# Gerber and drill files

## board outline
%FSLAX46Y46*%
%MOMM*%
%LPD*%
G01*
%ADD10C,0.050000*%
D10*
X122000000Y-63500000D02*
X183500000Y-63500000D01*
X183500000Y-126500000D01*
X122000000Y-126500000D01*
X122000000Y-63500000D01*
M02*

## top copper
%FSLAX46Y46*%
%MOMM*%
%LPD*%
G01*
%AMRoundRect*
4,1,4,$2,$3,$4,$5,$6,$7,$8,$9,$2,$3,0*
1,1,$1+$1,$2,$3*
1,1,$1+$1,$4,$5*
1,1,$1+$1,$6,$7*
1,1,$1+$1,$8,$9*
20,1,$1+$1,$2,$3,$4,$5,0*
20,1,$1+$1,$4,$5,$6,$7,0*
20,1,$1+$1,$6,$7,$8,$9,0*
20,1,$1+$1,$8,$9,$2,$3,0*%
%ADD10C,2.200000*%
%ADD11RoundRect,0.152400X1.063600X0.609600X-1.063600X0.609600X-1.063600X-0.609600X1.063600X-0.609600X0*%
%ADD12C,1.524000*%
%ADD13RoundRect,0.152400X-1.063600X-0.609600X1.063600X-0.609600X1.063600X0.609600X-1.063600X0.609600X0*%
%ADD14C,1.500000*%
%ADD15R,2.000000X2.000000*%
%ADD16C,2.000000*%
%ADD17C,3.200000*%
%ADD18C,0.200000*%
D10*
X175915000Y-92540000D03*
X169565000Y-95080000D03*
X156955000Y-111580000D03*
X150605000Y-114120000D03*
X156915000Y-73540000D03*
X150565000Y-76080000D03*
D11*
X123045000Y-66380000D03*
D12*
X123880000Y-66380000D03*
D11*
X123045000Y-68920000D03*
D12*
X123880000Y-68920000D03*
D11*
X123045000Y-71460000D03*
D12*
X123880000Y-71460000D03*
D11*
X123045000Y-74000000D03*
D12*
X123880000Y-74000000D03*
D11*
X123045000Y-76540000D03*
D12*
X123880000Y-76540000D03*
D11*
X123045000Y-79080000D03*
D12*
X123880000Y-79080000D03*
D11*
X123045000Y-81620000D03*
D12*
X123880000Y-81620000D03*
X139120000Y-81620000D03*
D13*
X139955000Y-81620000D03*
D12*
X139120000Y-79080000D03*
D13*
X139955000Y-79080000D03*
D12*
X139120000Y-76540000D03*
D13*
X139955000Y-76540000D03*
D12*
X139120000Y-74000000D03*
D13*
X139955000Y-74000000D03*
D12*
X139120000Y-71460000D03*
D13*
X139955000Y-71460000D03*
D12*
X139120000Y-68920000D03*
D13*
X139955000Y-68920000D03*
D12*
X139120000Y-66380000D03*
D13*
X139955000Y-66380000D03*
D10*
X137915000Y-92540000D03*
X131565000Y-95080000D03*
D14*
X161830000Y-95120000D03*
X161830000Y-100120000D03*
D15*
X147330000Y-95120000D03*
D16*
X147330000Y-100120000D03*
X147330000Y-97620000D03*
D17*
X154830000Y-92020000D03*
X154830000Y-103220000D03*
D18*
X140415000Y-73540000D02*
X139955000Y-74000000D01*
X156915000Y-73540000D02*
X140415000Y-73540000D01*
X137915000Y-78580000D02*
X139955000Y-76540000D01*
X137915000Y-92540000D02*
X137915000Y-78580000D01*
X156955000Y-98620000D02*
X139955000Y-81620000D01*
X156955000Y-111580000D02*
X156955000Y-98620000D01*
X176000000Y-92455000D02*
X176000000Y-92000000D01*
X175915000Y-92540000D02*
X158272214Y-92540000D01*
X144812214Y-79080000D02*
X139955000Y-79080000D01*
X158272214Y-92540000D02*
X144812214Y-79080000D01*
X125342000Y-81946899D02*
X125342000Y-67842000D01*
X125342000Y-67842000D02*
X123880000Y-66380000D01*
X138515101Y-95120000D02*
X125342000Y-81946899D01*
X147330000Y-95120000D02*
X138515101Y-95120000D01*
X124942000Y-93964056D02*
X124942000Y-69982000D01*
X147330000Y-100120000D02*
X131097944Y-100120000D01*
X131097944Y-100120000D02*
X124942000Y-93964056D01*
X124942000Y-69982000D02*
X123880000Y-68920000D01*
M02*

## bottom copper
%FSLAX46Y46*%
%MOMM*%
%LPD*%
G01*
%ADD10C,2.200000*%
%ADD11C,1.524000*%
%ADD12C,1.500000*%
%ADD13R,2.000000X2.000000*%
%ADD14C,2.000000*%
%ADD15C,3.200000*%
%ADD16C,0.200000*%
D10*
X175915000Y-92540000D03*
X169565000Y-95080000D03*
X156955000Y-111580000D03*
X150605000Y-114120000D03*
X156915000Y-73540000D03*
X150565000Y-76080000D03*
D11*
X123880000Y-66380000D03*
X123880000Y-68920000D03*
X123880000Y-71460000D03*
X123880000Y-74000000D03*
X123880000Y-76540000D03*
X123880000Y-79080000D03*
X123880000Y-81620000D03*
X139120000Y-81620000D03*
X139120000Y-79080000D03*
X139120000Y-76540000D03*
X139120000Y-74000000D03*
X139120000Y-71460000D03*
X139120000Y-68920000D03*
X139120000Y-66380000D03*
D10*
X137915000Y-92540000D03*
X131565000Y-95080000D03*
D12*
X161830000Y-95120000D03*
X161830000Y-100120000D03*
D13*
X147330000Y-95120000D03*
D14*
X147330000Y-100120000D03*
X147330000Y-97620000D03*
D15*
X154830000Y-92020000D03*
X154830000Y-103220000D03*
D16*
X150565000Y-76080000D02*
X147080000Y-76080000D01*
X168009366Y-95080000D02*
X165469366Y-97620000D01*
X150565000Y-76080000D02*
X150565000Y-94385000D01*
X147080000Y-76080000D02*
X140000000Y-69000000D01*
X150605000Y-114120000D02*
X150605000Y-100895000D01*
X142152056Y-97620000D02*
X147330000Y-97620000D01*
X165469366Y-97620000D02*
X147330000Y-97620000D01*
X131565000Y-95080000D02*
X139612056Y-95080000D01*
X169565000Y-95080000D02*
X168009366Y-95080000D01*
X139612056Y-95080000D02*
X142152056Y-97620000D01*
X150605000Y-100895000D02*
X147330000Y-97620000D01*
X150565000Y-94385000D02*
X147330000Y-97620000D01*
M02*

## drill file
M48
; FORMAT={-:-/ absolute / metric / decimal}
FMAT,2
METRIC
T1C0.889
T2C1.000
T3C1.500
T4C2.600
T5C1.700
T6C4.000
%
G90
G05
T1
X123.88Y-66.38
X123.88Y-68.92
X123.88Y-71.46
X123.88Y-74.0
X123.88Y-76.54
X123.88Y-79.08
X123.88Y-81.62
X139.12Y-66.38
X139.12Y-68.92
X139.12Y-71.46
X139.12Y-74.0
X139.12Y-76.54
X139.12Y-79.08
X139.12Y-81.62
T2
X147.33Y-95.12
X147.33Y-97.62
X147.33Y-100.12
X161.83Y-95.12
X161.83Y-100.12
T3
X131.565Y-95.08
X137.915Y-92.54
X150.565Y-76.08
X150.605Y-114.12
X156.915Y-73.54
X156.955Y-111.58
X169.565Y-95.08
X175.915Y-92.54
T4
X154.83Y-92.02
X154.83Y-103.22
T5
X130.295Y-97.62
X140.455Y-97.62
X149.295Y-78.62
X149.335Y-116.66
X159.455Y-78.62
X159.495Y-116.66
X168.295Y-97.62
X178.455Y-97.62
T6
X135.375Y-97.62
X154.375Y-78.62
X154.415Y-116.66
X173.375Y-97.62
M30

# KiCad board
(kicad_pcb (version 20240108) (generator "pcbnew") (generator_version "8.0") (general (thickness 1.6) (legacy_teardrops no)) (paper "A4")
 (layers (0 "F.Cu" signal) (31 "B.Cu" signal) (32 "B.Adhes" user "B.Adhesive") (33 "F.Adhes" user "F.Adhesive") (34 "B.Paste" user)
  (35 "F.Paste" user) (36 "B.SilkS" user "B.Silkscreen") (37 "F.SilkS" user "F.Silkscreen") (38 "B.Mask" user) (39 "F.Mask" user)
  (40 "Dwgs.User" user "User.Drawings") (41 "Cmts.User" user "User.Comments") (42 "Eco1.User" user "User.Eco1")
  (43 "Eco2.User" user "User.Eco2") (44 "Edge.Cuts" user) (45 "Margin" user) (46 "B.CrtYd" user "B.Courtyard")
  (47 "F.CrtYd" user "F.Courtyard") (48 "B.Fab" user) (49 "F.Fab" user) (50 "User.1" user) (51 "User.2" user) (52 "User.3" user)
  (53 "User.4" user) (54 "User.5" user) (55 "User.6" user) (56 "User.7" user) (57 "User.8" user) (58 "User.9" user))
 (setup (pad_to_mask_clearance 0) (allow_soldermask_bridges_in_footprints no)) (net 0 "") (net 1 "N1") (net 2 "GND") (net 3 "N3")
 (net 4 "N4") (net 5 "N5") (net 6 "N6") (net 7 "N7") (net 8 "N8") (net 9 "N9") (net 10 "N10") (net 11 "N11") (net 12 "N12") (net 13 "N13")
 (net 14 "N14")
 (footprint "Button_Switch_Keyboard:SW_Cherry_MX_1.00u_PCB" (layer "F.Cu") (at 175.915 92.54)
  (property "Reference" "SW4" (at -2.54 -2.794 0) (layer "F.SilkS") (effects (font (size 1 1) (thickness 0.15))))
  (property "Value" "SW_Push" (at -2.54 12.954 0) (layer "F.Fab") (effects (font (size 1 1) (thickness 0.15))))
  (pad "" np_thru_hole circle (at -7.62 5.08) (size 1.7 1.7) (drill 1.7) (layers "*.Cu" "*.Mask"))
  (pad "" np_thru_hole circle (at -2.54 5.08) (size 4 4) (drill 4) (layers "*.Cu" "*.Mask"))
  (pad "" np_thru_hole circle (at 2.54 5.08) (size 1.7 1.7) (drill 1.7) (layers "*.Cu" "*.Mask"))
  (pad "1" thru_hole circle (at 0 0) (size 2.2 2.2) (drill 1.5) (layers "*.Cu" "*.Mask") (remove_unused_layers no) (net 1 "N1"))
  (pad "2" thru_hole circle (at -6.35 2.54) (size 2.2 2.2) (drill 1.5) (layers "*.Cu" "*.Mask") (remove_unused_layers no) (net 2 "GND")))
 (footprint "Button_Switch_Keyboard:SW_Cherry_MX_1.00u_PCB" (layer "F.Cu") (at 156.955 111.58)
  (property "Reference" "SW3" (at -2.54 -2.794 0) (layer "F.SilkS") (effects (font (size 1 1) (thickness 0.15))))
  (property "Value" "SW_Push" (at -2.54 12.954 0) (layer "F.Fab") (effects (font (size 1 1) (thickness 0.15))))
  (pad "" np_thru_hole circle (at -7.62 5.08) (size 1.7 1.7) (drill 1.7) (layers "*.Cu" "*.Mask"))
  (pad "" np_thru_hole circle (at -2.54 5.08) (size 4 4) (drill 4) (layers "*.Cu" "*.Mask"))
  (pad "" np_thru_hole circle (at 2.54 5.08) (size 1.7 1.7) (drill 1.7) (layers "*.Cu" "*.Mask"))
  (pad "1" thru_hole circle (at 0 0) (size 2.2 2.2) (drill 1.5) (layers "*.Cu" "*.Mask") (remove_unused_layers no) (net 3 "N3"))
  (pad "2" thru_hole circle (at -6.35 2.54) (size 2.2 2.2) (drill 1.5) (layers "*.Cu" "*.Mask") (remove_unused_layers no) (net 2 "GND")))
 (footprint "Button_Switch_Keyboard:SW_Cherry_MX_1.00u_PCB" (layer "F.Cu") (at 156.915 73.54)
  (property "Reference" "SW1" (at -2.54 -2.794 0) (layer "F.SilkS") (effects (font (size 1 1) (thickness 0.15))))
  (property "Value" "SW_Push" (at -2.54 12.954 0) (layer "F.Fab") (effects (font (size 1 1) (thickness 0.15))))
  (pad "" np_thru_hole circle (at -7.62 5.08) (size 1.7 1.7) (drill 1.7) (layers "*.Cu" "*.Mask"))
  (pad "" np_thru_hole circle (at -2.54 5.08) (size 4 4) (drill 4) (layers "*.Cu" "*.Mask"))
  (pad "" np_thru_hole circle (at 2.54 5.08) (size 1.7 1.7) (drill 1.7) (layers "*.Cu" "*.Mask"))
  (pad "1" thru_hole circle (at 0 0) (size 2.2 2.2) (drill 1.5) (layers "*.Cu" "*.Mask") (remove_unused_layers no) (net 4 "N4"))
  (pad "2" thru_hole circle (at -6.35 2.54) (size 2.2 2.2) (drill 1.5) (layers "*.Cu" "*.Mask") (remove_unused_layers no) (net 2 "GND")))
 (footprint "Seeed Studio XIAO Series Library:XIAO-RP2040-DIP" (layer "F.Cu") (at 131.5 74)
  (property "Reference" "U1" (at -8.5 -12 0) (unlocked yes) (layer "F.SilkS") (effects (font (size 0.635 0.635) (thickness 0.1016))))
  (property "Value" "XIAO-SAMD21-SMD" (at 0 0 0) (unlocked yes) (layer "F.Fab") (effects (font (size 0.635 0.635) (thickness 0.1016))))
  (pad "1" smd roundrect (at -8.455 -7.62 180) (size 2.432 1.524) (layers "F.Cu" "F.Mask") (roundrect_rratio 0.1) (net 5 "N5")
   (thermal_bridge_angle 45))
  (pad "1" thru_hole circle (at -7.62 -7.62 180) (size 1.524 1.524) (drill 0.889) (layers "*.Cu" "*.Mask") (remove_unused_layers no)
   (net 5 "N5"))
  (pad "2" smd roundrect (at -8.455 -5.08 180) (size 2.432 1.524) (layers "F.Cu" "F.Mask") (roundrect_rratio 0.1) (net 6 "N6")
   (thermal_bridge_angle 45))
  (pad "2" thru_hole circle (at -7.62 -5.08 180) (size 1.524 1.524) (drill 0.889) (layers "*.Cu" "*.Mask") (remove_unused_layers no)
   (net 6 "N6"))
  (pad "3" smd roundrect (at -8.455 -2.54 180) (size 2.432 1.524) (layers "F.Cu" "F.Mask") (roundrect_rratio 0.1) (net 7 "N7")
   (thermal_bridge_angle 45))
  (pad "3" thru_hole circle (at -7.62 -2.54 180) (size 1.524 1.524) (drill 0.889) (layers "*.Cu" "*.Mask") (remove_unused_layers no)
   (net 7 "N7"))
  (pad "4" smd roundrect (at -8.455 0 180) (size 2.432 1.524) (layers "F.Cu" "F.Mask") (roundrect_rratio 0.1) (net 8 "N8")
   (thermal_bridge_angle 45))
  (pad "4" thru_hole circle (at -7.62 0 180) (size 1.524 1.524) (drill 0.889) (layers "*.Cu" "*.Mask") (remove_unused_layers no)
   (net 8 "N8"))
  (pad "5" smd roundrect (at -8.455 2.54 180) (size 2.432 1.524) (layers "F.Cu" "F.Mask") (roundrect_rratio 0.1) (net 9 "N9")
   (thermal_bridge_angle 45))
  (pad "5" thru_hole circle (at -7.62 2.54 180) (size 1.524 1.524) (drill 0.889) (layers "*.Cu" "*.Mask") (remove_unused_layers no)
   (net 9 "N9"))
  (pad "6" smd roundrect (at -8.455 5.08 180) (size 2.432 1.524) (layers "F.Cu" "F.Mask") (roundrect_rratio 0.1) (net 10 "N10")
   (thermal_bridge_angle 45))
  (pad "6" thru_hole circle (at -7.62 5.08 180) (size 1.524 1.524) (drill 0.889) (layers "*.Cu" "*.Mask") (remove_unused_layers no)
   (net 10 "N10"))
  (pad "7" smd roundrect (at -8.455 7.62 180) (size 2.432 1.524) (layers "F.Cu" "F.Mask") (roundrect_rratio 0.1) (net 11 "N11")
   (thermal_bridge_angle 45))
  (pad "7" thru_hole circle (at -7.62 7.62 180) (size 1.524 1.524) (drill 0.889) (layers "*.Cu" "*.Mask") (remove_unused_layers no)
   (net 11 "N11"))
  (pad "8" thru_hole circle (at 7.62 7.62) (size 1.524 1.524) (drill 0.889) (layers "*.Cu" "*.Mask") (remove_unused_layers no) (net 3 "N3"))
  (pad "8" smd roundrect (at 8.455 7.62) (size 2.432 1.524) (layers "F.Cu" "F.Mask") (roundrect_rratio 0.1) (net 3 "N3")
   (thermal_bridge_angle 45))
  (pad "9" thru_hole circle (at 7.62 5.08) (size 1.524 1.524) (drill 0.889) (layers "*.Cu" "*.Mask") (remove_unused_layers no) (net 1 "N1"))
  (pad "9" smd roundrect (at 8.455 5.08) (size 2.432 1.524) (layers "F.Cu" "F.Mask") (roundrect_rratio 0.1) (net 1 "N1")
   (thermal_bridge_angle 45))
  (pad "10" thru_hole circle (at 7.62 2.54) (size 1.524 1.524) (drill 0.889) (layers "*.Cu" "*.Mask") (remove_unused_layers no)
   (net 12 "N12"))
  (pad "10" smd roundrect (at 8.455 2.54) (size 2.432 1.524) (layers "F.Cu" "F.Mask") (roundrect_rratio 0.1) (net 12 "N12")
   (thermal_bridge_angle 45))
  (pad "11" thru_hole circle (at 7.62 0) (size 1.524 1.524) (drill 0.889) (layers "*.Cu" "*.Mask") (remove_unused_layers no) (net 4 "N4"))
  (pad "11" smd roundrect (at 8.455 0) (size 2.432 1.524) (layers "F.Cu" "F.Mask") (roundrect_rratio 0.1) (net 4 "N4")
   (thermal_bridge_angle 45))
  (pad "12" thru_hole circle (at 7.62 -2.54) (size 1.524 1.524) (drill 0.889) (layers "*.Cu" "*.Mask") (remove_unused_layers no)
   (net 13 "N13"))
  (pad "12" smd roundrect (at 8.455 -2.54) (size 2.432 1.524) (layers "F.Cu" "F.Mask") (roundrect_rratio 0.1) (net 13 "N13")
   (thermal_bridge_angle 45))
  (pad "13" thru_hole circle (at 7.62 -5.08) (size 1.524 1.524) (drill 0.889) (layers "*.Cu" "*.Mask") (remove_unused_layers no)
   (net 2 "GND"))
  (pad "13" smd roundrect (at 8.455 -5.08) (size 2.432 1.524) (layers "F.Cu" "F.Mask") (roundrect_rratio 0.1) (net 2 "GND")
   (thermal_bridge_angle 45))
  (pad "14" thru_hole circle (at 7.62 -7.62) (size 1.524 1.524) (drill 0.889) (layers "*.Cu" "*.Mask") (remove_unused_layers no)
   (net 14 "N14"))
  (pad "14" smd roundrect (at 8.455 -7.62) (size 2.432 1.524) (layers "F.Cu" "F.Mask") (roundrect_rratio 0.1) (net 14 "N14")
   (thermal_bridge_angle 45)))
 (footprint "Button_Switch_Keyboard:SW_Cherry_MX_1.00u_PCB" (layer "F.Cu") (at 137.915 92.54)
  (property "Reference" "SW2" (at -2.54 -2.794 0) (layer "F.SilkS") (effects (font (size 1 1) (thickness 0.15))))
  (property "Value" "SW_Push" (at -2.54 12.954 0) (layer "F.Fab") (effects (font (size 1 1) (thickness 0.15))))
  (pad "" np_thru_hole circle (at -7.62 5.08) (size 1.7 1.7) (drill 1.7) (layers "*.Cu" "*.Mask"))
  (pad "" np_thru_hole circle (at -2.54 5.08) (size 4 4) (drill 4) (layers "*.Cu" "*.Mask"))
  (pad "" np_thru_hole circle (at 2.54 5.08) (size 1.7 1.7) (drill 1.7) (layers "*.Cu" "*.Mask"))
  (pad "1" thru_hole circle (at 0 0) (size 2.2 2.2) (drill 1.5) (layers "*.Cu" "*.Mask") (remove_unused_layers no) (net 12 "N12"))
  (pad "2" thru_hole circle (at -6.35 2.54) (size 2.2 2.2) (drill 1.5) (layers "*.Cu" "*.Mask") (remove_unused_layers no) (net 2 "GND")))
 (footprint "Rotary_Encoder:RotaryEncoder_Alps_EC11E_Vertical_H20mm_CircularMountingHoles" (layer "F.Cu") (at 147.33 95.12)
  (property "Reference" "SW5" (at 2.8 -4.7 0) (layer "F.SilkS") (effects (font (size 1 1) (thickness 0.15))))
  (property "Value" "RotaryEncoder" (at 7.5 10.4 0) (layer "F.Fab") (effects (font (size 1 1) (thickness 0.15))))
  (pad "" thru_hole circle (at 14.5 0) (size 1.5 1.5) (drill 1) (layers "*.Cu" "*.Mask") (remove_unused_layers no))
  (pad "" thru_hole circle (at 14.5 5) (size 1.5 1.5) (drill 1) (layers "*.Cu" "*.Mask") (remove_unused_layers no))
  (pad "A" thru_hole rect (at 0 0) (size 2 2) (drill 1) (layers "*.Cu" "*.Mask") (remove_unused_layers no) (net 5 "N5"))
  (pad "B" thru_hole circle (at 0 5) (size 2 2) (drill 1) (layers "*.Cu" "*.Mask") (remove_unused_layers no) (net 6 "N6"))
  (pad "C" thru_hole circle (at 0 2.5) (size 2 2) (drill 1) (layers "*.Cu" "*.Mask") (remove_unused_layers no) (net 2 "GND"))
  (pad "MP" thru_hole circle (at 7.5 -3.1) (size 3.2 3.2) (drill 2.6) (layers "*.Cu" "*.Mask") (remove_unused_layers no))
  (pad "MP" thru_hole circle (at 7.5 8.1) (size 3.2 3.2) (drill 2.6) (layers "*.Cu" "*.Mask") (remove_unused_layers no)))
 (gr_rect (start 122 63.5) (end 183.5 126.5) (stroke (width 0.05) (type default)) (fill none) (layer "Edge.Cuts"))
 (segment (start 140.415 73.54) (end 139.955 74) (width 0.2) (layer "F.Cu") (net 4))
 (segment (start 156.915 73.54) (end 140.415 73.54) (width 0.2) (layer "F.Cu") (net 4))
 (segment (start 150.565 76.08) (end 147.08 76.08) (width 0.2) (layer "B.Cu") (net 2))
 (segment (start 168.009366 95.08) (end 165.469366 97.62) (width 0.2) (layer "B.Cu") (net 2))
 (segment (start 150.565 76.08) (end 150.565 94.385) (width 0.2) (layer "B.Cu") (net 2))
 (segment (start 147.08 76.08) (end 140 69) (width 0.2) (layer "B.Cu") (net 2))
 (segment (start 150.605 114.12) (end 150.605 100.895) (width 0.2) (layer "B.Cu") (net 2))
 (segment (start 142.152056 97.62) (end 147.33 97.62) (width 0.2) (layer "B.Cu") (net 2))
 (segment (start 165.469366 97.62) (end 147.33 97.62) (width 0.2) (layer "B.Cu") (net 2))
 (segment (start 131.565 95.08) (end 139.612056 95.08) (width 0.2) (layer "B.Cu") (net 2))
 (segment (start 169.565 95.08) (end 168.009366 95.08) (width 0.2) (layer "B.Cu") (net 2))
 (segment (start 139.612056 95.08) (end 142.152056 97.62) (width 0.2) (layer "B.Cu") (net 2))
 (segment (start 150.605 100.895) (end 147.33 97.62) (width 0.2) (layer "B.Cu") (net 2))
 (segment (start 150.565 94.385) (end 147.33 97.62) (width 0.2) (layer "B.Cu") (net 2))
 (segment (start 137.915 78.58) (end 139.955 76.54) (width 0.2) (layer "F.Cu") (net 12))
 (segment (start 137.915 92.54) (end 137.915 78.58) (width 0.2) (layer "F.Cu") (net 12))
 (segment (start 156.955 98.62) (end 139.955 81.62) (width 0.2) (layer "F.Cu") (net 3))
 (segment (start 156.955 111.58) (end 156.955 98.62) (width 0.2) (layer "F.Cu") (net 3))
 (segment (start 176 92.455) (end 176 92) (width 0.2) (layer "F.Cu") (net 1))
 (segment (start 175.915 92.54) (end 158.272214 92.54) (width 0.2) (layer "F.Cu") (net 1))
 (segment (start 144.812214 79.08) (end 139.955 79.08) (width 0.2) (layer "F.Cu") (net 1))
 (segment (start 158.272214 92.54) (end 144.812214 79.08) (width 0.2) (layer "F.Cu") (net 1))
 (segment (start 125.342 81.946899) (end 125.342 67.842) (width 0.2) (layer "F.Cu") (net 5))
 (segment (start 125.342 67.842) (end 123.88 66.38) (width 0.2) (layer "F.Cu") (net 5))
 (segment (start 138.515101 95.12) (end 125.342 81.946899) (width 0.2) (layer "F.Cu") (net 5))
 (segment (start 147.33 95.12) (end 138.515101 95.12) (width 0.2) (layer "F.Cu") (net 5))
 (segment (start 124.942 93.964056) (end 124.942 69.982) (width 0.2) (layer "F.Cu") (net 6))
 (segment (start 147.33 100.12) (end 131.097944 100.12) (width 0.2) (layer "F.Cu") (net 6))
 (segment (start 131.097944 100.12) (end 124.942 93.964056) (width 0.2) (layer "F.Cu") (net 6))
 (segment (start 124.942 69.982) (end 123.88 68.92) (width 0.2) (layer "F.Cu") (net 6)))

